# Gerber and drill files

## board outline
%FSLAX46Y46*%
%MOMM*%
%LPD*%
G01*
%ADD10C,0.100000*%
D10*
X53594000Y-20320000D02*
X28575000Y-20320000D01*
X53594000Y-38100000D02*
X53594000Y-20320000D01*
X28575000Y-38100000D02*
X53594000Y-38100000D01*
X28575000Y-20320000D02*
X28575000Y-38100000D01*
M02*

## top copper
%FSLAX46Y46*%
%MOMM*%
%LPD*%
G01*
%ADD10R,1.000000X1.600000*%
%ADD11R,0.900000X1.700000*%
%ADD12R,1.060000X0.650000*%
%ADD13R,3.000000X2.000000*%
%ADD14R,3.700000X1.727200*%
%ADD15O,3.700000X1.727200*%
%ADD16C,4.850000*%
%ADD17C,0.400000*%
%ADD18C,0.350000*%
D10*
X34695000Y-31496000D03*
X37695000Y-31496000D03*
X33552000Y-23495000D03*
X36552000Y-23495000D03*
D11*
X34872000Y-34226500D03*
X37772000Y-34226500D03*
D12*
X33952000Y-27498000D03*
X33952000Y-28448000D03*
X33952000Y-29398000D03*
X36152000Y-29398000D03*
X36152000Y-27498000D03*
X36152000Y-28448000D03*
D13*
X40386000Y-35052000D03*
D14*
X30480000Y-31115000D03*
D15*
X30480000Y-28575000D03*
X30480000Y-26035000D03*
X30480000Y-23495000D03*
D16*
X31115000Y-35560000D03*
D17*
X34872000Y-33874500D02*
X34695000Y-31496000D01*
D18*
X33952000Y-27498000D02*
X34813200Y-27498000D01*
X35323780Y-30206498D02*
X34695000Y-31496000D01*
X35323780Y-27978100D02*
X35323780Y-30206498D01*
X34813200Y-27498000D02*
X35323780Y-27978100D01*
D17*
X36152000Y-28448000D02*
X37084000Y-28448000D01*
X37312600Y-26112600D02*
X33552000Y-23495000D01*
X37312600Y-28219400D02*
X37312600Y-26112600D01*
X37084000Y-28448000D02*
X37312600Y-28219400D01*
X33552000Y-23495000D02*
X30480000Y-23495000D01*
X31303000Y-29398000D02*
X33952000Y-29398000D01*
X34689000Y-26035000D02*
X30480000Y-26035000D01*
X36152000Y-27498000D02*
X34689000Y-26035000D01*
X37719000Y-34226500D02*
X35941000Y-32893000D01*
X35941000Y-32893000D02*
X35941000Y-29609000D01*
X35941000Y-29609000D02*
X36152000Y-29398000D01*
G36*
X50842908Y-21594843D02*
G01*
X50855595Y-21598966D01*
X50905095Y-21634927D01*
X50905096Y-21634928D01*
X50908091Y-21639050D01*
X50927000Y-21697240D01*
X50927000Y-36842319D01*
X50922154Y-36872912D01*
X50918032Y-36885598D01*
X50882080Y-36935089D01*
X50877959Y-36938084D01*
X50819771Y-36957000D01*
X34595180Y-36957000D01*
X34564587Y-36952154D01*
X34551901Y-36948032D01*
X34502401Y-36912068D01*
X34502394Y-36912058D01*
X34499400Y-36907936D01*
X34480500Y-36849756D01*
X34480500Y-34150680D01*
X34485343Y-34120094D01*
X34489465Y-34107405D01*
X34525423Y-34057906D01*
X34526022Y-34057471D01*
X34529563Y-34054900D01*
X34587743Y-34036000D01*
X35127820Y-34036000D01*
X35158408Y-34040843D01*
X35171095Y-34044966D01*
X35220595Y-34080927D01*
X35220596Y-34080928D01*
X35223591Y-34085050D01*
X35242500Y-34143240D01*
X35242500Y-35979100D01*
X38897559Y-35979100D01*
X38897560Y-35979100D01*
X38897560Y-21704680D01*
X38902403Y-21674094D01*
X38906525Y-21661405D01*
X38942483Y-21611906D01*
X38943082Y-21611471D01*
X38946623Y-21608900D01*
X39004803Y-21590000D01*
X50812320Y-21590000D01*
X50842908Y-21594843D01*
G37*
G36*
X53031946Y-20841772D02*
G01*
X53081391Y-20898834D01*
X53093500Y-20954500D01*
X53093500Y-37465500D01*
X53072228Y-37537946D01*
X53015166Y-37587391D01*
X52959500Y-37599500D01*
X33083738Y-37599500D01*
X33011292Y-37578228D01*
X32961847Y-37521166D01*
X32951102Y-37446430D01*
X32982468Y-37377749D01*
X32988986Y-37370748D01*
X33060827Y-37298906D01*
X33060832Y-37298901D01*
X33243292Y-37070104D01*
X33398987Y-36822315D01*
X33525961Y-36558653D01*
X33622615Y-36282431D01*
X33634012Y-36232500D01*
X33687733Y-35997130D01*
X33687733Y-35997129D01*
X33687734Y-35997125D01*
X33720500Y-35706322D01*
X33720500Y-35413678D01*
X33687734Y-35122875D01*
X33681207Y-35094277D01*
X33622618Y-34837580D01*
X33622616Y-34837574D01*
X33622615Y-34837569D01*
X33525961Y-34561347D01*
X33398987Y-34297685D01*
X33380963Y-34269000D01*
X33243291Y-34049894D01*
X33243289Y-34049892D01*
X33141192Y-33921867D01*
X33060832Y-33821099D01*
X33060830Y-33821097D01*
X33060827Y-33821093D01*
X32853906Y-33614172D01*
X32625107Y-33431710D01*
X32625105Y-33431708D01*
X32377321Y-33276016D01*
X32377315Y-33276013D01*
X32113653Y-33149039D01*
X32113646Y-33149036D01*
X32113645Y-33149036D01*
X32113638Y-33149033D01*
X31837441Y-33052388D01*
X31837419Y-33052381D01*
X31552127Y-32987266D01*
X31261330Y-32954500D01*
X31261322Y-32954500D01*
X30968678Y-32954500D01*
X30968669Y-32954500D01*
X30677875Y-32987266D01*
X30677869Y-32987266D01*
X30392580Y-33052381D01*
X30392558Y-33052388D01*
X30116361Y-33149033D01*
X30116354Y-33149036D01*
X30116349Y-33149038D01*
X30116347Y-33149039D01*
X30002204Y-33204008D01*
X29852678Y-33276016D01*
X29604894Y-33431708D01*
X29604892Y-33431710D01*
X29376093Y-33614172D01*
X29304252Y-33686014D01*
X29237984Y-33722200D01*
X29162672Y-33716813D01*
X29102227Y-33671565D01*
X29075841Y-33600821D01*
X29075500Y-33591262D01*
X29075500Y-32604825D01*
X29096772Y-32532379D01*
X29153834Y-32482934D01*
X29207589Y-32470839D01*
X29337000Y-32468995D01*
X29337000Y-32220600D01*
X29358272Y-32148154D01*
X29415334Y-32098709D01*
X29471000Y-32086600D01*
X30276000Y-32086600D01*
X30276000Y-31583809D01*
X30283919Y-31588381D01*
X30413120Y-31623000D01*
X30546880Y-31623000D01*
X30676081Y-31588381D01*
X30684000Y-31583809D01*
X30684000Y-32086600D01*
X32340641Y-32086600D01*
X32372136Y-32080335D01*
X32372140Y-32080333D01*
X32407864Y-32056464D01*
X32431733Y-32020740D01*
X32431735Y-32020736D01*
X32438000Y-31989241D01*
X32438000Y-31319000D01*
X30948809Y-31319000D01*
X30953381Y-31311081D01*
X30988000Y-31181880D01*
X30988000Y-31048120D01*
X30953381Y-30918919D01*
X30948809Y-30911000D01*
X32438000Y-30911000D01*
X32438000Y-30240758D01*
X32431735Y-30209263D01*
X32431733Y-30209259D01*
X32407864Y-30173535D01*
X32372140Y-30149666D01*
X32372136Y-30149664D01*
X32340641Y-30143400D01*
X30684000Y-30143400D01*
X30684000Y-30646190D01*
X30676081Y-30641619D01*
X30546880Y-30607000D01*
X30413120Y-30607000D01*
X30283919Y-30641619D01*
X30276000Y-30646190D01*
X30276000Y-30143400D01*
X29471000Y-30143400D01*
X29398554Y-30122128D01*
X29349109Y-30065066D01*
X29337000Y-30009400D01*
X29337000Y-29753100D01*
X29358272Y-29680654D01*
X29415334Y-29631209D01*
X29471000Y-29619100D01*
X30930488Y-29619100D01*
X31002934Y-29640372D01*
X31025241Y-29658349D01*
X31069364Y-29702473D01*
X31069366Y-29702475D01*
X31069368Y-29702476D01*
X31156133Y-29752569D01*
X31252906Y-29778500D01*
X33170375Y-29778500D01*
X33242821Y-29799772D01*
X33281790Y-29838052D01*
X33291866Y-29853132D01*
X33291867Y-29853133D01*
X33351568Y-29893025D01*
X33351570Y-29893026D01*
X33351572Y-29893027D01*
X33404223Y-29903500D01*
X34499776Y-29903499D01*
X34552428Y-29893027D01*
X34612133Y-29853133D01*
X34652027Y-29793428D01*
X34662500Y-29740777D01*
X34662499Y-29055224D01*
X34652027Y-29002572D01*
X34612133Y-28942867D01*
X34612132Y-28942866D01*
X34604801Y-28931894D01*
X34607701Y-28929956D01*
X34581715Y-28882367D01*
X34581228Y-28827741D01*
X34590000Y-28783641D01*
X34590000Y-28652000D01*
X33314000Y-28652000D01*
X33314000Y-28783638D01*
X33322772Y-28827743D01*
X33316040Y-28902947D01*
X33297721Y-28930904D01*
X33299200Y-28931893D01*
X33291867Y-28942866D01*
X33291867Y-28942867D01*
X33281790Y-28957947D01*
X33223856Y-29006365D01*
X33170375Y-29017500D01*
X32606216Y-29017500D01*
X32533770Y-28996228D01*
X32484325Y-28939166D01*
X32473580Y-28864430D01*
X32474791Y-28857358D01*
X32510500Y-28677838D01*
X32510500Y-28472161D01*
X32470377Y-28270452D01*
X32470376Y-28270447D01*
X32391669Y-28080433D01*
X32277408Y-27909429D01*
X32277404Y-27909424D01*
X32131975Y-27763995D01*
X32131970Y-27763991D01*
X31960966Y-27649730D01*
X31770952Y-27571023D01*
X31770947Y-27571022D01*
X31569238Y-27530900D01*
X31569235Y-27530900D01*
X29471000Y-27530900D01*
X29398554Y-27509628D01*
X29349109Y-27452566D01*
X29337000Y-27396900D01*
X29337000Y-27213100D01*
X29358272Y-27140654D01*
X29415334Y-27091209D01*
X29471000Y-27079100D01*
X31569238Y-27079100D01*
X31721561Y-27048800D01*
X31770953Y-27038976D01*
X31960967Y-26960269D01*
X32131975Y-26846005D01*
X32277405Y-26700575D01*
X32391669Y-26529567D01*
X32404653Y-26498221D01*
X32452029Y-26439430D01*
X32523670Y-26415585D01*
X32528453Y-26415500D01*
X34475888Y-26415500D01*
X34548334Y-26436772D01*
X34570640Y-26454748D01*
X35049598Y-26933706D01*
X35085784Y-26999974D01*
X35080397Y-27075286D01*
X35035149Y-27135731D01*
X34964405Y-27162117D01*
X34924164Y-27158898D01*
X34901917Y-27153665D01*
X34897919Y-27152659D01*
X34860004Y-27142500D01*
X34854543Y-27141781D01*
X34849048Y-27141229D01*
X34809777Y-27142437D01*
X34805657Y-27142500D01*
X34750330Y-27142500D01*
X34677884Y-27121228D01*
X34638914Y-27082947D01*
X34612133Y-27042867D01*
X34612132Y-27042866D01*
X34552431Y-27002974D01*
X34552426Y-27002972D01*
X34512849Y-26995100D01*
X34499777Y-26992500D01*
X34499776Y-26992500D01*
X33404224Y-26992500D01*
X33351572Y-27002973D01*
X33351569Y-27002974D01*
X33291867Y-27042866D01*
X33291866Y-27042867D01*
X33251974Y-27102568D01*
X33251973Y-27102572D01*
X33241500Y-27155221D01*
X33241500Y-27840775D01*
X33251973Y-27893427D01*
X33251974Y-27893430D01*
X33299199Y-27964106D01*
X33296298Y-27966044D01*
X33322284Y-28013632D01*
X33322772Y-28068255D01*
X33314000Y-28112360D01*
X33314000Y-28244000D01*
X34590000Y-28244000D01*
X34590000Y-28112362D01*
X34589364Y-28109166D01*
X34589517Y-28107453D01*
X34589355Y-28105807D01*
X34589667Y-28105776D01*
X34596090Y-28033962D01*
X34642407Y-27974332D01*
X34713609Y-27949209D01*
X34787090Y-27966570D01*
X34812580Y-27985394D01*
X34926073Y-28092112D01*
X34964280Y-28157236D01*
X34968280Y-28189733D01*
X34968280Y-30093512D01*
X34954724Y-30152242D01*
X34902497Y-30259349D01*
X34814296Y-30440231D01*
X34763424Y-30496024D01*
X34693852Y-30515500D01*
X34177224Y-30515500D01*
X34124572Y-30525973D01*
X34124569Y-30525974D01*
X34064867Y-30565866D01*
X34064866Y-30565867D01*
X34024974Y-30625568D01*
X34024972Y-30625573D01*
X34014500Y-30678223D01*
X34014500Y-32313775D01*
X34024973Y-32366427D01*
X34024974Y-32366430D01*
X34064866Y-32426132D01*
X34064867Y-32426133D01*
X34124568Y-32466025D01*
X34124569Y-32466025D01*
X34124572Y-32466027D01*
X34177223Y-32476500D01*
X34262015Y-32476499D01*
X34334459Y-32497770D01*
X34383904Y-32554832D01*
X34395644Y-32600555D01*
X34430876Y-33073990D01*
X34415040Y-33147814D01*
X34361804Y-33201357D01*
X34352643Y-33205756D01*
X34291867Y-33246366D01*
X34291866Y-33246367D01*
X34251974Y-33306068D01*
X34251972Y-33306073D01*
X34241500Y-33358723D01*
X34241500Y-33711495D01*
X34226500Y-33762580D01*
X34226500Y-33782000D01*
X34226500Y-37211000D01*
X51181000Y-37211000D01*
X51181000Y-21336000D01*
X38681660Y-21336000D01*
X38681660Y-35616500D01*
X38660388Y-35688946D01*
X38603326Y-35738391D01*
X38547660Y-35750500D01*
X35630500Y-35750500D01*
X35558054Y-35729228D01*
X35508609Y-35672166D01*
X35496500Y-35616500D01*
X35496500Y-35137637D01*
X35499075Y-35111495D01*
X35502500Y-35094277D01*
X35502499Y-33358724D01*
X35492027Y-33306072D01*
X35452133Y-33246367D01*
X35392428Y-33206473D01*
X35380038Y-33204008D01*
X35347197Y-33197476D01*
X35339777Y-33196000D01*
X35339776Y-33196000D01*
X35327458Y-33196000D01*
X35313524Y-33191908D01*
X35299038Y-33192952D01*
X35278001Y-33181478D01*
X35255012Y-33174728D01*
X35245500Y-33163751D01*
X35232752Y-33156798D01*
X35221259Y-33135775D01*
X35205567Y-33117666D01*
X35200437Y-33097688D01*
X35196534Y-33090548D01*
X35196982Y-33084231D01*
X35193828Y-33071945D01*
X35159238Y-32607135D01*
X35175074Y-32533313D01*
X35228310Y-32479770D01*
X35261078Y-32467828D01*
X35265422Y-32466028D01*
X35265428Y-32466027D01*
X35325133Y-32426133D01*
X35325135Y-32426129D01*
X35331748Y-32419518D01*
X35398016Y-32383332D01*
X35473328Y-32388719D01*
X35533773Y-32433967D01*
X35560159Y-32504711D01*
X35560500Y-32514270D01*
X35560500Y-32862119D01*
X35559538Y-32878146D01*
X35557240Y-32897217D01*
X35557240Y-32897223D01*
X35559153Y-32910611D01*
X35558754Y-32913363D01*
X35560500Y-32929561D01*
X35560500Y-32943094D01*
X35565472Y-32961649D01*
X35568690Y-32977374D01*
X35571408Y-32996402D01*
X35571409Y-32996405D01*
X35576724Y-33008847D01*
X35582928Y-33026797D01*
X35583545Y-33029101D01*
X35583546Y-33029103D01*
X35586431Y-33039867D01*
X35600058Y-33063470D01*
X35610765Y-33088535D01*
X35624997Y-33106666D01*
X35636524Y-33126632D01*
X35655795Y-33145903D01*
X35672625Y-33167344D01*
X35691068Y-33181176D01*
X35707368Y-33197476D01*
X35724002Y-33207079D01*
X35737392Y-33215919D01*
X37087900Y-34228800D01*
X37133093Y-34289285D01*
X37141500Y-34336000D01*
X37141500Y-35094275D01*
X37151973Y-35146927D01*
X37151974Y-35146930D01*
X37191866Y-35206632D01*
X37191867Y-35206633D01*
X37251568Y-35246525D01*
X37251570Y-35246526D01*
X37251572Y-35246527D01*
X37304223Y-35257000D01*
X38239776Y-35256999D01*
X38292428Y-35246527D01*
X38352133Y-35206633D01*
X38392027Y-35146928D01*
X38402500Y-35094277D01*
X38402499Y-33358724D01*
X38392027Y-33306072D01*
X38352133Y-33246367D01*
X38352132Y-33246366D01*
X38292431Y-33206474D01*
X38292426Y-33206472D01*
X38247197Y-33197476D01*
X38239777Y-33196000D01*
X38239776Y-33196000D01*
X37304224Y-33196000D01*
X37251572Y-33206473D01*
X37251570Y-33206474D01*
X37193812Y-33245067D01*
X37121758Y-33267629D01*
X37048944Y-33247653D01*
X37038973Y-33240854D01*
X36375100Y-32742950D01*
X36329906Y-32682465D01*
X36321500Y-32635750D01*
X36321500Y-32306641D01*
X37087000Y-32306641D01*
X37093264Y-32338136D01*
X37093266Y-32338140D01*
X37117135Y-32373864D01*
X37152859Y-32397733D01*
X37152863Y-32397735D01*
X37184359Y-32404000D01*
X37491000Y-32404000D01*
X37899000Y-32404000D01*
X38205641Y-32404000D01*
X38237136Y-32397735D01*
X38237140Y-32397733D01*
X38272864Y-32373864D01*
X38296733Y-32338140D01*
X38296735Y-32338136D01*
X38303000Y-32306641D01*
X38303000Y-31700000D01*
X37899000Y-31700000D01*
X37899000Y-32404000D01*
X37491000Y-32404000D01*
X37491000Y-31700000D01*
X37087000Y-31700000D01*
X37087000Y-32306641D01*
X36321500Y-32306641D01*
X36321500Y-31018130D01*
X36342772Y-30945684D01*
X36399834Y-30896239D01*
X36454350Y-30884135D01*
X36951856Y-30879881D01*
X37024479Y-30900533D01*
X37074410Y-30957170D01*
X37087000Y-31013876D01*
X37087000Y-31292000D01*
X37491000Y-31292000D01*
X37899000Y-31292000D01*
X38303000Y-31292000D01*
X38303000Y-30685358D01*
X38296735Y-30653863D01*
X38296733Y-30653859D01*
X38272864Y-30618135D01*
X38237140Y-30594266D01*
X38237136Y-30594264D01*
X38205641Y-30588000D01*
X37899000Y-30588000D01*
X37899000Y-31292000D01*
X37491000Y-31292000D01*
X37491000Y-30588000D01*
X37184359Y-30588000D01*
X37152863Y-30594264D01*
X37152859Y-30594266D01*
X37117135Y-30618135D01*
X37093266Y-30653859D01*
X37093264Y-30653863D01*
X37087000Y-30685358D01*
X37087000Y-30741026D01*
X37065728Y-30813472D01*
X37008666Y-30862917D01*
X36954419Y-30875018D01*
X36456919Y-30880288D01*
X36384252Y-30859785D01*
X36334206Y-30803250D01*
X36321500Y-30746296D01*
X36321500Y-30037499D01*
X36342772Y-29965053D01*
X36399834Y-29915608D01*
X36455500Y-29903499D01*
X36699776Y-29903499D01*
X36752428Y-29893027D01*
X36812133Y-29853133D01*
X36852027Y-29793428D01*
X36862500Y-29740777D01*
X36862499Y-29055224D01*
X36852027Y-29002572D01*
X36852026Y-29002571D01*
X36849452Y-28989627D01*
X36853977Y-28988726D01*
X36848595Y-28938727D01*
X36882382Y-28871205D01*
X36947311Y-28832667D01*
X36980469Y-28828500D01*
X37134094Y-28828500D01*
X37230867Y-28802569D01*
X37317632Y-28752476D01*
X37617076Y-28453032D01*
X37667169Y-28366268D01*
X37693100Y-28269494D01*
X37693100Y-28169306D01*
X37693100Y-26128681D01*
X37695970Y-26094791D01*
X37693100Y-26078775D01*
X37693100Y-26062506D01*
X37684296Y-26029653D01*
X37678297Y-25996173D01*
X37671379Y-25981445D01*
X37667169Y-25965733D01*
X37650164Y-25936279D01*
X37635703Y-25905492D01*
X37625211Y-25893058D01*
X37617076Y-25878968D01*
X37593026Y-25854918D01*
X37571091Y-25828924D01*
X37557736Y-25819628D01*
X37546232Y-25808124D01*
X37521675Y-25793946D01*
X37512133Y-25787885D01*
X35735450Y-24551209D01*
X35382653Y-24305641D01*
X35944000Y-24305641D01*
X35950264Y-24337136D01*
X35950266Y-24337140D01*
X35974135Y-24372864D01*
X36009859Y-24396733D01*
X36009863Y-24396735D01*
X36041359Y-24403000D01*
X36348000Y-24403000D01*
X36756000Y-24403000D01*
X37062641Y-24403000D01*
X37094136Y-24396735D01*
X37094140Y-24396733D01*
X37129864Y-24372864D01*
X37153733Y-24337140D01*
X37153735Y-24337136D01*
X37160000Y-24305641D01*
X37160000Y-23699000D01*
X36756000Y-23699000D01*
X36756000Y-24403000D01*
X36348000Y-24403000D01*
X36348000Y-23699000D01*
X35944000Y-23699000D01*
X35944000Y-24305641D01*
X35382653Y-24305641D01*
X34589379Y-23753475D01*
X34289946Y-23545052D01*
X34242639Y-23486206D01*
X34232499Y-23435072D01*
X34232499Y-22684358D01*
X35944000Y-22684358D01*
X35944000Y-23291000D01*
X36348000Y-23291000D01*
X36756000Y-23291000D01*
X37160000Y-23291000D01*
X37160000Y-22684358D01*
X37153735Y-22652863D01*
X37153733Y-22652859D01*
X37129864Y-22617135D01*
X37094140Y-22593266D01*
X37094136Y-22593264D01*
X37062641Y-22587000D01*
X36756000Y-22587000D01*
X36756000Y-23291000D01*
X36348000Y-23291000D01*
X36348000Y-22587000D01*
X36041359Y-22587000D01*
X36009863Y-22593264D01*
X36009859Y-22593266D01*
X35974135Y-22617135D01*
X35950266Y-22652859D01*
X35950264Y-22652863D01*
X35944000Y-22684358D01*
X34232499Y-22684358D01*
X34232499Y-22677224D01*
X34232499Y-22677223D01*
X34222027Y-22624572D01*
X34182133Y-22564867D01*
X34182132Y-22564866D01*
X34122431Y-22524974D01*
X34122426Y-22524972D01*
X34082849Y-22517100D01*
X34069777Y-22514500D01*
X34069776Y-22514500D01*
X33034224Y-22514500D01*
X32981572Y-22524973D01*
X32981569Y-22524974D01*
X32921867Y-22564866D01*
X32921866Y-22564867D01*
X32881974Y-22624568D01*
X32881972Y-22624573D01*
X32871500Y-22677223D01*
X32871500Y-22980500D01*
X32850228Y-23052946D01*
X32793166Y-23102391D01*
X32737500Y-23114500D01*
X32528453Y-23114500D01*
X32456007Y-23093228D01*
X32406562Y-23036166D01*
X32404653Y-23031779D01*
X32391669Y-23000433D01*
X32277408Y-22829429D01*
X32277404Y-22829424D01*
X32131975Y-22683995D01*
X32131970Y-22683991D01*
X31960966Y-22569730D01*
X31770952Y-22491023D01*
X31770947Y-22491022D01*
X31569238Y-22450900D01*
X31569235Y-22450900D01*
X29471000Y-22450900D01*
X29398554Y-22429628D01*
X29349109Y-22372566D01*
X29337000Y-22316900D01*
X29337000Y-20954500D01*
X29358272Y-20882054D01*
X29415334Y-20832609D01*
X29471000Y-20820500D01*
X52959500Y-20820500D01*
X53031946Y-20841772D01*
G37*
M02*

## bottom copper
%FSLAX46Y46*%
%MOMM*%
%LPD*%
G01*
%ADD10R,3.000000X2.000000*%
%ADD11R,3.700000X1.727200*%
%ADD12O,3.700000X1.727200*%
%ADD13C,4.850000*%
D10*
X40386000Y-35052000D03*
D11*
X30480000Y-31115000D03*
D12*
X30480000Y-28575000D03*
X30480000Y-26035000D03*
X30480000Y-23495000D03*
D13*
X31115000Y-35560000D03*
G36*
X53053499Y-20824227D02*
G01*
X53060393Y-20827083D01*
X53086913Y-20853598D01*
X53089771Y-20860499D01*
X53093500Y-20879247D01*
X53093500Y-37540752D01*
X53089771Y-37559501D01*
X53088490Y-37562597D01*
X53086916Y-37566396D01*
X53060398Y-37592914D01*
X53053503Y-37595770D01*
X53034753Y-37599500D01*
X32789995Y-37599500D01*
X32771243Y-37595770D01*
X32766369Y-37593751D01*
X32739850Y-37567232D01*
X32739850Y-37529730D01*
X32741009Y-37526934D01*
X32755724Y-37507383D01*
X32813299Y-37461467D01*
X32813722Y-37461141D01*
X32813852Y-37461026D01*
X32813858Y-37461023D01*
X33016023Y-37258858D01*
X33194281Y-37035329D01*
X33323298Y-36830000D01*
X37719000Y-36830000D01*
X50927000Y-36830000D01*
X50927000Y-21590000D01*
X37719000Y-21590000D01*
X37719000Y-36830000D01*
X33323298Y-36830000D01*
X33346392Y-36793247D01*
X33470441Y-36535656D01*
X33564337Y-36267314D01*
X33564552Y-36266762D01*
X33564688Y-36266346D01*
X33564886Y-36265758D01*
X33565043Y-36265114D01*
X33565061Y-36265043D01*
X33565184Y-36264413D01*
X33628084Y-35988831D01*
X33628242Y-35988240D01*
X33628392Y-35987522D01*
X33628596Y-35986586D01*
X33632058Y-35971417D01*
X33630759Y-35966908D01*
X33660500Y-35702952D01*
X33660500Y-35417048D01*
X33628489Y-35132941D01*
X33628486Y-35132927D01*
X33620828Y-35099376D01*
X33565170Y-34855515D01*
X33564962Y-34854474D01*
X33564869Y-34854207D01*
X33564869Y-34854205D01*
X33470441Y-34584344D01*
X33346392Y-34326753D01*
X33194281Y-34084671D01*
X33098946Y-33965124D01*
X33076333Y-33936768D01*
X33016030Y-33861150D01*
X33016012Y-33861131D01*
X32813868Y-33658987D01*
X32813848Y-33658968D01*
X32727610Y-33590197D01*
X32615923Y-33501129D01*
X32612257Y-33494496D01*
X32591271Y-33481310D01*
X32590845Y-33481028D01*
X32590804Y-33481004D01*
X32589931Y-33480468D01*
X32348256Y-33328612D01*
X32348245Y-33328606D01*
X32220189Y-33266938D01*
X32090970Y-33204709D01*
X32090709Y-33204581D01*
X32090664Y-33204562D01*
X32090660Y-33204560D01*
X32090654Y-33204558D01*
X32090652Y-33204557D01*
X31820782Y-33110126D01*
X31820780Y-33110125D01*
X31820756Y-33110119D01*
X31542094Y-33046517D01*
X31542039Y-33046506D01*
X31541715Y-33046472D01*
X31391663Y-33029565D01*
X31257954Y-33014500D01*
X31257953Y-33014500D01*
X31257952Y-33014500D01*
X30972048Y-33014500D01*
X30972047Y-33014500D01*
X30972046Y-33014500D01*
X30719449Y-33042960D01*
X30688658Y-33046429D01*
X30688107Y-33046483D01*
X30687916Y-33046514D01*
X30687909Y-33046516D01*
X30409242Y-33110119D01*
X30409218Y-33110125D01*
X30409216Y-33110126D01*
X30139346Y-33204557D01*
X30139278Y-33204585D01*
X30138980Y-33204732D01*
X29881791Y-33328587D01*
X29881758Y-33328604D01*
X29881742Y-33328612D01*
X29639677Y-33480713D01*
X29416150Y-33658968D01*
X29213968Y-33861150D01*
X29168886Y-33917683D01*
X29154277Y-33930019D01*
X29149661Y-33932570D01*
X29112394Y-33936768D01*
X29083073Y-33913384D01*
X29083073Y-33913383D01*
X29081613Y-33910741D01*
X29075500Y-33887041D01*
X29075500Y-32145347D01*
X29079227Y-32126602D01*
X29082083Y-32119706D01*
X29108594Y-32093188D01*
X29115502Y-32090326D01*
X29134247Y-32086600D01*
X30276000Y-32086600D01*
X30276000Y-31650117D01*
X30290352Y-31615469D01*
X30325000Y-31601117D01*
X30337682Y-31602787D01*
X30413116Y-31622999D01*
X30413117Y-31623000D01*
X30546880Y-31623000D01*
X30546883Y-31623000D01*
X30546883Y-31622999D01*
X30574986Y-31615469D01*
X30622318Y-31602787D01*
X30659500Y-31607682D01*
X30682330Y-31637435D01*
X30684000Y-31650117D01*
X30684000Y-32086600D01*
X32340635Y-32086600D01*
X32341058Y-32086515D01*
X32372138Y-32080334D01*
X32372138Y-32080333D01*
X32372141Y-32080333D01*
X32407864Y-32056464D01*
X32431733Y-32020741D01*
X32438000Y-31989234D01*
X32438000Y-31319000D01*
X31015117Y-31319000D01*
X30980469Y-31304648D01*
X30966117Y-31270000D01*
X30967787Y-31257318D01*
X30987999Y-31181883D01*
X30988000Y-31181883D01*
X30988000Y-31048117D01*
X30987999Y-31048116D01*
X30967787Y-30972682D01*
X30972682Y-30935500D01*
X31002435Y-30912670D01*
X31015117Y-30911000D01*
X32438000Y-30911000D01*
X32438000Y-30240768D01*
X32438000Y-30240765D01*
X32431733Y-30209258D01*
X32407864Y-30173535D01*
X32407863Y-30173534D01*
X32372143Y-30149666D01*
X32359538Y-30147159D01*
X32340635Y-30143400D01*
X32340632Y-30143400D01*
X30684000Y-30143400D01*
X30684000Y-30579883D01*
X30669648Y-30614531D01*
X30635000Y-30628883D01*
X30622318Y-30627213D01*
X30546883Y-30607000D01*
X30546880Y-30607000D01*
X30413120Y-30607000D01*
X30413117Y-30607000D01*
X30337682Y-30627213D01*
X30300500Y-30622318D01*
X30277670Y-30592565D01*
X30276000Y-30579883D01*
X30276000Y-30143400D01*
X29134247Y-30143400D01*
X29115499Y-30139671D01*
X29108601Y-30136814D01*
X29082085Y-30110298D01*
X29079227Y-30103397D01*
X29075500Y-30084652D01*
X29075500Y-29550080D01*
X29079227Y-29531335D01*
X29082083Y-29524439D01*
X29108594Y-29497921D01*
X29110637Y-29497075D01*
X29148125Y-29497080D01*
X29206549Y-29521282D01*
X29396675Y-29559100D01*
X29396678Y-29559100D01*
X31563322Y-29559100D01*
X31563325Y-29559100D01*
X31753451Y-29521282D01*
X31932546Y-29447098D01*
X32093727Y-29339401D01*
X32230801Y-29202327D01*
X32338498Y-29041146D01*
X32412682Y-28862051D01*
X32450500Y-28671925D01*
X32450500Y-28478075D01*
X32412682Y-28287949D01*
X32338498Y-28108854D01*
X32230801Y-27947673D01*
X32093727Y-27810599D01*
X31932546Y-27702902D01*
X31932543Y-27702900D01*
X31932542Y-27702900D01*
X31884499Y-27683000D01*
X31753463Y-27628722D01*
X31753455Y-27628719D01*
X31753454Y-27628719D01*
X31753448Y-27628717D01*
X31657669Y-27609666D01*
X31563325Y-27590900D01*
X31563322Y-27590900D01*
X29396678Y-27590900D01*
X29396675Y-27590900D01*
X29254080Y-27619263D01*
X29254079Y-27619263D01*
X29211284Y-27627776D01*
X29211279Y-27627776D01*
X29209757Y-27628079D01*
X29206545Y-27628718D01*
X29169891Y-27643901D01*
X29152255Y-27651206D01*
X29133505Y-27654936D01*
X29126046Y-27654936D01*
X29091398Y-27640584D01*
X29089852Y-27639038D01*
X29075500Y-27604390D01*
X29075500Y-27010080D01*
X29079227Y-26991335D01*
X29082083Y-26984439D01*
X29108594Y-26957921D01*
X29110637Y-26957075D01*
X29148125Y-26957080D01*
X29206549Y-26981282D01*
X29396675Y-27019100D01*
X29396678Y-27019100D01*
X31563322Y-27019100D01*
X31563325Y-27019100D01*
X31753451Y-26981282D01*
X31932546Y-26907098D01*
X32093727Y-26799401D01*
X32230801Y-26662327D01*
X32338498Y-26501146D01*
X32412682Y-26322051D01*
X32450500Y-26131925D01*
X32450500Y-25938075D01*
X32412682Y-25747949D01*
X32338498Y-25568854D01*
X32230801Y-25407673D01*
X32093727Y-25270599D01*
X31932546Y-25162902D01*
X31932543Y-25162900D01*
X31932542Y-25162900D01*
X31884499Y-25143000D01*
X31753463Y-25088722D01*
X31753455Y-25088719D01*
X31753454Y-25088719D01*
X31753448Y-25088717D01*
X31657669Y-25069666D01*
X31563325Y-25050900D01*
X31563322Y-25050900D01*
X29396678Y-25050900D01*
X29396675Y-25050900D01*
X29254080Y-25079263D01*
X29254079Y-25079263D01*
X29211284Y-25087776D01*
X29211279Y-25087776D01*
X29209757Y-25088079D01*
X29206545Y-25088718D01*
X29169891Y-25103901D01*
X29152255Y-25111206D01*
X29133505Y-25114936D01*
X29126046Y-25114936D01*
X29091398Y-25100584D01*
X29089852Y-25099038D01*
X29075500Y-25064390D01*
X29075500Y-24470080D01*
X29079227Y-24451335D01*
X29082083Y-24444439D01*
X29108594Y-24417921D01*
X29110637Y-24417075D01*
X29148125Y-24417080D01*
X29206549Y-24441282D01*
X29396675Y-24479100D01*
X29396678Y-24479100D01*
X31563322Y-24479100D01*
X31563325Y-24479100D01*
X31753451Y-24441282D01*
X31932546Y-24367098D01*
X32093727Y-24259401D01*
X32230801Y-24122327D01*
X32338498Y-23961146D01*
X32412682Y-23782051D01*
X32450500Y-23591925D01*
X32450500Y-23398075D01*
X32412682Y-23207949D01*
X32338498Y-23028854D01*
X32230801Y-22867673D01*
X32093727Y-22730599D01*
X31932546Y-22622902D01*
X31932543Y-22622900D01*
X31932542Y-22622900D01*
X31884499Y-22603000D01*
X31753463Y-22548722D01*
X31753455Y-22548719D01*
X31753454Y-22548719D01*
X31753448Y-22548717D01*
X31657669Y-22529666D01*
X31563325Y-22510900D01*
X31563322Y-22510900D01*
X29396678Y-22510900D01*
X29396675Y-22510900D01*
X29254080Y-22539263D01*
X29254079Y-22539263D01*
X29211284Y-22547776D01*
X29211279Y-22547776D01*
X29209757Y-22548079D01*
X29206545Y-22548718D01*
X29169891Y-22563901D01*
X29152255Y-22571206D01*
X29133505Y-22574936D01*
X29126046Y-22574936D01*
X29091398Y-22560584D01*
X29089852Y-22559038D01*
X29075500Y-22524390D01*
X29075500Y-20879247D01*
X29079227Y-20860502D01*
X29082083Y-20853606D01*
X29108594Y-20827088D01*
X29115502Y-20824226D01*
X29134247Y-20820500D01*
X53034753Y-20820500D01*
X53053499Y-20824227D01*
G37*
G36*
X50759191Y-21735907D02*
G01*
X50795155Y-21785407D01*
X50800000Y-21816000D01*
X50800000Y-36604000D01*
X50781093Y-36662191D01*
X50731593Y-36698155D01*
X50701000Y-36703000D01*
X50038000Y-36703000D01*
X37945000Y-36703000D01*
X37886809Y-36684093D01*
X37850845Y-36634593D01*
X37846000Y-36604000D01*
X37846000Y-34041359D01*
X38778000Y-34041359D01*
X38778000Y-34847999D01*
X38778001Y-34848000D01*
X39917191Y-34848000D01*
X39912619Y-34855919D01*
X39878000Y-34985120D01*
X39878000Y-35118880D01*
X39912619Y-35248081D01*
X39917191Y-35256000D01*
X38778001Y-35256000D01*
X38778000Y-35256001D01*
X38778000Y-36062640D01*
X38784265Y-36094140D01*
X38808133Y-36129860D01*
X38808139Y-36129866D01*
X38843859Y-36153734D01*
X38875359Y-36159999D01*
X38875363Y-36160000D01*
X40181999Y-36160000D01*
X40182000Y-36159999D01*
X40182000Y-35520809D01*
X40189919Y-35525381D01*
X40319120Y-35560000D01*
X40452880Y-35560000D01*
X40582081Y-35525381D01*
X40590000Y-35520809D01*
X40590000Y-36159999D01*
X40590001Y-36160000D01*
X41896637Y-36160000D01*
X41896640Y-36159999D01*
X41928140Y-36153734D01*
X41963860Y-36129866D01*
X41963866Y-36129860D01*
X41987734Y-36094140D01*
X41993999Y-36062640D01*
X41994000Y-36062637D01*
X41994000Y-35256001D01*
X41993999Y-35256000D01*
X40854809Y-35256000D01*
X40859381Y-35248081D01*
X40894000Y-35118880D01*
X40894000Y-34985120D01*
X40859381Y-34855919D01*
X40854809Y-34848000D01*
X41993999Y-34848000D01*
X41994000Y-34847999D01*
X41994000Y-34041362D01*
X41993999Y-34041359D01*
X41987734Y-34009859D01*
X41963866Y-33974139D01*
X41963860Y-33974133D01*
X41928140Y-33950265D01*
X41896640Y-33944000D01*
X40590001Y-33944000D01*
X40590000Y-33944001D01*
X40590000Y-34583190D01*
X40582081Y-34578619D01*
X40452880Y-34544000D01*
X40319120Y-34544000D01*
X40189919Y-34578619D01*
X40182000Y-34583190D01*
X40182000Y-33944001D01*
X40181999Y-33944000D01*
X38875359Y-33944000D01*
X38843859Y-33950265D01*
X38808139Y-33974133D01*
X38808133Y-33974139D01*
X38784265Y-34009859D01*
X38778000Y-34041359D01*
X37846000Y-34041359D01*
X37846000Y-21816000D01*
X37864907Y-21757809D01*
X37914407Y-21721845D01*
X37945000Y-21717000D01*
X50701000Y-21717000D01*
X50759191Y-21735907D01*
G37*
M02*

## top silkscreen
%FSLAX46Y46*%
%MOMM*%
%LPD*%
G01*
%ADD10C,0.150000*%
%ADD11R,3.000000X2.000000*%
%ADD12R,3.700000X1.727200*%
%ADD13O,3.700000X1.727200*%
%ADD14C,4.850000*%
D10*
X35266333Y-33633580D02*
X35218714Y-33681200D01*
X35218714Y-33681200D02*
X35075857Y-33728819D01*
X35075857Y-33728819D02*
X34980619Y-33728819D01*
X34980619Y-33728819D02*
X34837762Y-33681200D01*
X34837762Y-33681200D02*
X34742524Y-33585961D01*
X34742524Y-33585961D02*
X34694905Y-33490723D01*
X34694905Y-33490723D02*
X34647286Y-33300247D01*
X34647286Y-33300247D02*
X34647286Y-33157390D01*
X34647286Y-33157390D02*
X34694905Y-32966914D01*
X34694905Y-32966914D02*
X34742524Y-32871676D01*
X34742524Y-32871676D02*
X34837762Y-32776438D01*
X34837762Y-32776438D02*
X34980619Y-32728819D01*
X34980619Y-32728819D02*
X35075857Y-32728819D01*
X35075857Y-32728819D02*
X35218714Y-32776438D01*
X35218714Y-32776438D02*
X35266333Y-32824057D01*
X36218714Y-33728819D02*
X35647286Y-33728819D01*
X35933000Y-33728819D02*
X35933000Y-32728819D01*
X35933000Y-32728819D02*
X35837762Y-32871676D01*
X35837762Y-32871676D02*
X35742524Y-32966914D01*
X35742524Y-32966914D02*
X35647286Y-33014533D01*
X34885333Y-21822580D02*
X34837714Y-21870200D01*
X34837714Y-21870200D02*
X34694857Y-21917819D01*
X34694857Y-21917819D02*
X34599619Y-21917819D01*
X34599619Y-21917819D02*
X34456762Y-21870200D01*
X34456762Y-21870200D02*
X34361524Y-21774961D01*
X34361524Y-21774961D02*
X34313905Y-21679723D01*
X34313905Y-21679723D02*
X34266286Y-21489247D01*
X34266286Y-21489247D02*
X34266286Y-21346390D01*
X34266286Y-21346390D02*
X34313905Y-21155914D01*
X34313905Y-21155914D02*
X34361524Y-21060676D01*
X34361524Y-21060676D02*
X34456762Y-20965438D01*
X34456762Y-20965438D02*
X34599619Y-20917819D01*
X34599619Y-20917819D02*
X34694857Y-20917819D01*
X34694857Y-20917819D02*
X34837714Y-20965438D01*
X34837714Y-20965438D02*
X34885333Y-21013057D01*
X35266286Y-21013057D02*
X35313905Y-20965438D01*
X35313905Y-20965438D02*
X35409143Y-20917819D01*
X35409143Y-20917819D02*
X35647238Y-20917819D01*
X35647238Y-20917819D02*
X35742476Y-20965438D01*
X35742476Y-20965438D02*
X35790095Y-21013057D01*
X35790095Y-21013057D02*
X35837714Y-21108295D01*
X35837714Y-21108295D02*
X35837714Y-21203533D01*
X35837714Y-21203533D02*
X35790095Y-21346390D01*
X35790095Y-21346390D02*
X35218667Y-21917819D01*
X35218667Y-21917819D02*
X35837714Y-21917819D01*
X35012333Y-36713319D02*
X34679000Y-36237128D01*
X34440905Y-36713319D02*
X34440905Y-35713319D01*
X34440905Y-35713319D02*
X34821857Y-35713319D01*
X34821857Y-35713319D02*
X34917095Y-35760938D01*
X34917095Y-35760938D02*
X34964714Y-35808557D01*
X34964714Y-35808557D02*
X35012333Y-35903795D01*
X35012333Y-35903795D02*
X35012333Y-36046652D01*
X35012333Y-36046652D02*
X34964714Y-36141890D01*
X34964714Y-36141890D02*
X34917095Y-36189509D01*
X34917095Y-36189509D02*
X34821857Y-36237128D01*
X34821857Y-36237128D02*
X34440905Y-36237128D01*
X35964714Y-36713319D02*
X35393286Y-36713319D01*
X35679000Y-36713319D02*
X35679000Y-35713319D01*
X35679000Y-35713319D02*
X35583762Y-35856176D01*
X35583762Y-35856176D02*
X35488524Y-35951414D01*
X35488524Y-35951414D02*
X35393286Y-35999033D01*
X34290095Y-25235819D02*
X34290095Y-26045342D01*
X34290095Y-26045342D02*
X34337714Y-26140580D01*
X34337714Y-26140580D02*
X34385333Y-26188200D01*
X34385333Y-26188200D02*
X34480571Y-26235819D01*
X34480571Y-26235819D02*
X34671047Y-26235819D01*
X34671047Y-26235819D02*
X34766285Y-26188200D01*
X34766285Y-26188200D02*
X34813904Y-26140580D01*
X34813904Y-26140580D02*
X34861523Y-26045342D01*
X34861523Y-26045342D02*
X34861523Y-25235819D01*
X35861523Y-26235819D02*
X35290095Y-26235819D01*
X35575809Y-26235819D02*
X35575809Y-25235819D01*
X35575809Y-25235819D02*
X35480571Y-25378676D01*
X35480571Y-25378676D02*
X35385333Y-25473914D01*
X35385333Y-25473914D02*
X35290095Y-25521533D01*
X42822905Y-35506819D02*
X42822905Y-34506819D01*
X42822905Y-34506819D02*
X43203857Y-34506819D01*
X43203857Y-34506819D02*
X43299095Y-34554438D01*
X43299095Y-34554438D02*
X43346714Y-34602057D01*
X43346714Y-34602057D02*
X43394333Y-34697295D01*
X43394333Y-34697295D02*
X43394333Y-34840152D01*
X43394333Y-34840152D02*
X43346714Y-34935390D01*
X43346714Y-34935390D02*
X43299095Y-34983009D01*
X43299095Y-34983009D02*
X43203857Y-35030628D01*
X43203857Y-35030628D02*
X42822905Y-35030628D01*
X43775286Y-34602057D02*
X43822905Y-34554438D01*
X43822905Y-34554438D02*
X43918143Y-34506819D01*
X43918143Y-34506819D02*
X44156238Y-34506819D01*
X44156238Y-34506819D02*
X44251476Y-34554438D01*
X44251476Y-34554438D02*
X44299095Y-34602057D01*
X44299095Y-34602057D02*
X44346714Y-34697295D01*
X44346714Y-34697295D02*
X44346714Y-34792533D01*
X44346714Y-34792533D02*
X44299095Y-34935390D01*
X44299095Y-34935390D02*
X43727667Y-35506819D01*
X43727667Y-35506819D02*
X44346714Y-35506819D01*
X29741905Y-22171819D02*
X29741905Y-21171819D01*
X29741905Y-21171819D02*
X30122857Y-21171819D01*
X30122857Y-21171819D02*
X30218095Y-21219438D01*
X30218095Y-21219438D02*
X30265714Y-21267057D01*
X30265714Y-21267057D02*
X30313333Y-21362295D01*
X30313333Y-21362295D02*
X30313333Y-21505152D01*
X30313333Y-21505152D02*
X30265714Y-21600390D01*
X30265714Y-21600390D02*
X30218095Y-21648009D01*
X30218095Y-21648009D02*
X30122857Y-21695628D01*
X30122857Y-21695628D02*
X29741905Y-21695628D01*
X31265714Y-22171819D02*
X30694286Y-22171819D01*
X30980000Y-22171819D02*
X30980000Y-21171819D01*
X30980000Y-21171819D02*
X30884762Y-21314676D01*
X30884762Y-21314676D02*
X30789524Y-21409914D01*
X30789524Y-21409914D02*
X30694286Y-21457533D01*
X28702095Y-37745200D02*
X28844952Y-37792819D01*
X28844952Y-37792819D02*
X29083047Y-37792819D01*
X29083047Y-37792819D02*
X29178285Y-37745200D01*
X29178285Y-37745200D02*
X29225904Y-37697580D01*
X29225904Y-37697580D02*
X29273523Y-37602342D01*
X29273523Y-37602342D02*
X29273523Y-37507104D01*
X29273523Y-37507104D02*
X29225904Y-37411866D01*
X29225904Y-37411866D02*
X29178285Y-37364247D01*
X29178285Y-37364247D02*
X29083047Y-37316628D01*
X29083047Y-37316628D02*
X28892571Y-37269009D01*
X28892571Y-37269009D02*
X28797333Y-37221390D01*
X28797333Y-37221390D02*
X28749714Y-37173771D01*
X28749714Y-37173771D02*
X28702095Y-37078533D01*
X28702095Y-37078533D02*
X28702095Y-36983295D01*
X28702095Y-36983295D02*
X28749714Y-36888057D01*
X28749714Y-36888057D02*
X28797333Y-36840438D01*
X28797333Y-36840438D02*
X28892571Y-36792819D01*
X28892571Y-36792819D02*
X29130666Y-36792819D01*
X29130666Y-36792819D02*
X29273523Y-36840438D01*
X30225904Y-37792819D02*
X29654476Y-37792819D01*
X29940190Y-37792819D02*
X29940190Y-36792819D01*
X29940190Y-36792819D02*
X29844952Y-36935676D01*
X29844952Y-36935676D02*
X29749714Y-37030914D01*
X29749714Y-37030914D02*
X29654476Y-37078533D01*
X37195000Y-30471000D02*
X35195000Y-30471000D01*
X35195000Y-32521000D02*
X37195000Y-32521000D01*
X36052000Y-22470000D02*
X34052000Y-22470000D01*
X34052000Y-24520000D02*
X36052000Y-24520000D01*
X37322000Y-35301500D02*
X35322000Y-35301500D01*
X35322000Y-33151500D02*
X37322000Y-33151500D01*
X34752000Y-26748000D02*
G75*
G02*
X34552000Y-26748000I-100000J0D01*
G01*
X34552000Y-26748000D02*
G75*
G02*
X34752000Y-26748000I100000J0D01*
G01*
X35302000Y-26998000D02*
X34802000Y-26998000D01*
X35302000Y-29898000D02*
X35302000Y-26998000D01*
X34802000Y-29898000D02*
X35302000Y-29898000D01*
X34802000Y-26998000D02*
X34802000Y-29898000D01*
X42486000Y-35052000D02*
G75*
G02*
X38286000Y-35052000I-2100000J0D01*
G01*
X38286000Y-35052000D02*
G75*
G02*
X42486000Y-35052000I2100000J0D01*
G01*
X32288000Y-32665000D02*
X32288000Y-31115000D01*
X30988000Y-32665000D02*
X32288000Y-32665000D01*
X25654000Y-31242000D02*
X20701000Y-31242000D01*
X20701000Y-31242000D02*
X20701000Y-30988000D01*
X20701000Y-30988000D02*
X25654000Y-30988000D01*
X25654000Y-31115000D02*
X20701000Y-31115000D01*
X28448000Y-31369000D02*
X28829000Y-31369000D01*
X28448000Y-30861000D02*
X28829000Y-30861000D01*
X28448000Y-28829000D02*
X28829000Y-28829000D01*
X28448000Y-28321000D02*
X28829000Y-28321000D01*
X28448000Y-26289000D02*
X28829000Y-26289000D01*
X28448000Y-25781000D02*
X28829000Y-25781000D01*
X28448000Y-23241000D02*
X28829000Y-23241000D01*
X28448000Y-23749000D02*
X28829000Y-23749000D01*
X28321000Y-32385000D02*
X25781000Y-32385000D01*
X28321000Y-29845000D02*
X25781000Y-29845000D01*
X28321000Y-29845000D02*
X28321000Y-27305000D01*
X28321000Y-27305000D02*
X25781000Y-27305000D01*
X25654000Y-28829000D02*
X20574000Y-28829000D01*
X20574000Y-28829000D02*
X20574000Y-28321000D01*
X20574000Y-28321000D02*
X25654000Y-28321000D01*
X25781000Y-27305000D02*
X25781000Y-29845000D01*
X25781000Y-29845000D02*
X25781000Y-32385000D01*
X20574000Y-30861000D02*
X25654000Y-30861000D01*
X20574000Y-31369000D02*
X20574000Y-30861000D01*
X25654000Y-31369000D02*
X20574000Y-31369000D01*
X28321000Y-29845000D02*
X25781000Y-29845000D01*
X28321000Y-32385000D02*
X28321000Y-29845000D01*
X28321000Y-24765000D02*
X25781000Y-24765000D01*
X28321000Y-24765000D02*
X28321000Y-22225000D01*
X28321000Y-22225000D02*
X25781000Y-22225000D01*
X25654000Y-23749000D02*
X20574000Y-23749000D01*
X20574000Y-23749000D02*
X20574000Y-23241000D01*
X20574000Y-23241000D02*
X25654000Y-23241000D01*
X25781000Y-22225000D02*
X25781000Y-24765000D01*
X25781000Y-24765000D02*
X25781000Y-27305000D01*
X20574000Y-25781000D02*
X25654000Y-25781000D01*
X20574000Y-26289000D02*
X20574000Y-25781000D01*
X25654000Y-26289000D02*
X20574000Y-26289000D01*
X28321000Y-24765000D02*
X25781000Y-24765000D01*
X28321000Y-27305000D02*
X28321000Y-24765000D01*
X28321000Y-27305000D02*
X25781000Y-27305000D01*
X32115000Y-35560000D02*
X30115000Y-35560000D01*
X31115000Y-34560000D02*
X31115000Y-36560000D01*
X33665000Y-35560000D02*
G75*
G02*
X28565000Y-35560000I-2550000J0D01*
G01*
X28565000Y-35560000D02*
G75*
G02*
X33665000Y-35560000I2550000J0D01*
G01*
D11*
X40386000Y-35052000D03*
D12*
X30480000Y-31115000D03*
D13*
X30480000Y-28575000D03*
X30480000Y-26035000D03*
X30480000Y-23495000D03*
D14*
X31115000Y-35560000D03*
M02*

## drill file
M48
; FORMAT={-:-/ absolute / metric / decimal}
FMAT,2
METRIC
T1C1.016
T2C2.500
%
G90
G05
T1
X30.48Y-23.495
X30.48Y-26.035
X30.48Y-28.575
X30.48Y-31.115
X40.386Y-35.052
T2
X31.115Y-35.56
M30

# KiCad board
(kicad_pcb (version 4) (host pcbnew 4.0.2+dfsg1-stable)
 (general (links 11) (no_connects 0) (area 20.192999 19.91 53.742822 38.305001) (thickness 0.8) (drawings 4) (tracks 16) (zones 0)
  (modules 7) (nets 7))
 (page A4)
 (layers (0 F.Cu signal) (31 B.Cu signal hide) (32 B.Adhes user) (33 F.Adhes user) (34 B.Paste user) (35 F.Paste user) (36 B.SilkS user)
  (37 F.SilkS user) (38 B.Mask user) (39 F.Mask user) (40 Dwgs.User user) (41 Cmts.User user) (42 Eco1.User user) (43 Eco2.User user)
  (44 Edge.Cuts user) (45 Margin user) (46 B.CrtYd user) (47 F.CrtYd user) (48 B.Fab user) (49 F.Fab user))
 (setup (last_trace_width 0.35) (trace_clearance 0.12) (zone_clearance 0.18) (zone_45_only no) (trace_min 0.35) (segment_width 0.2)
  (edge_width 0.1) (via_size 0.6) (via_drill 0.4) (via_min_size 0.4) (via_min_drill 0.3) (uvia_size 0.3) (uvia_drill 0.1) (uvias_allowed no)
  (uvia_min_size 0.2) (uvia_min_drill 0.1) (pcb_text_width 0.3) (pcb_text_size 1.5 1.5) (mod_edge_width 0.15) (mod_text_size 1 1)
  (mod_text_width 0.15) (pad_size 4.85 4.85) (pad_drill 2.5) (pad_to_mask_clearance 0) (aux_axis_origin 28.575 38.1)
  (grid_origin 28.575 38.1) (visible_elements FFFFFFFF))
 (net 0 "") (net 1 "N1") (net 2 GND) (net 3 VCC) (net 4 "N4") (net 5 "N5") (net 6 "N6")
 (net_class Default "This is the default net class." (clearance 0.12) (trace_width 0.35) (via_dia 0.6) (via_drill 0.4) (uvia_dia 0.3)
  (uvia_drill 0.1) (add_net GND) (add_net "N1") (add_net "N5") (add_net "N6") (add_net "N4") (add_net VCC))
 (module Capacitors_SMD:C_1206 (layer F.Cu) (at 36.195 31.496)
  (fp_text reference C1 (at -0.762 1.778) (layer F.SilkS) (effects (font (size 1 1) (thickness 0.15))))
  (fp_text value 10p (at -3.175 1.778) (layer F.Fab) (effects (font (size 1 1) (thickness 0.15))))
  (fp_line (start 1 -1.025) (end -1 -1.025) (layer F.SilkS) (width 0.15))
  (fp_line (start -1 1.025) (end 1 1.025) (layer F.SilkS) (width 0.15))
  (pad 1 smd rect (at -1.5 0) (size 1 1.6) (layers F.Cu F.Paste F.Mask) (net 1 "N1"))
  (pad 2 smd rect (at 1.5 0) (size 1 1.6) (layers F.Cu F.Paste F.Mask) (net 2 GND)))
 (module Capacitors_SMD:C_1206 (layer F.Cu) (at 35.052 23.495)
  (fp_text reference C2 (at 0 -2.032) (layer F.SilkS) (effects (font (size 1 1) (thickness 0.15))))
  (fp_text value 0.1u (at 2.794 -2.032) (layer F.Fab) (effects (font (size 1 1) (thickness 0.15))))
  (fp_line (start 1 -1.025) (end -1 -1.025) (layer F.SilkS) (width 0.15))
  (fp_line (start -1 1.025) (end 1 1.025) (layer F.SilkS) (width 0.15))
  (pad 1 smd rect (at -1.5 0) (size 1 1.6) (layers F.Cu F.Paste F.Mask) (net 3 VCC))
  (pad 2 smd rect (at 1.5 0) (size 1 1.6) (layers F.Cu F.Paste F.Mask) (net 2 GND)))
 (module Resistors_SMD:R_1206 (layer F.Cu) (at 36.322 34.2265)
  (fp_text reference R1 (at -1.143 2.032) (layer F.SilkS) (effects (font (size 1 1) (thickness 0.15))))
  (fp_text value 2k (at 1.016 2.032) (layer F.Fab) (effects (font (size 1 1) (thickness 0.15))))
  (fp_line (start 1 1.075) (end -1 1.075) (layer F.SilkS) (width 0.15))
  (fp_line (start -1 -1.075) (end 1 -1.075) (layer F.SilkS) (width 0.15))
  (pad 1 smd rect (at -1.45 0) (size 0.9 1.7) (layers F.Cu F.Paste F.Mask) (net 1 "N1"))
  (pad 2 smd rect (at 1.45 0) (size 0.9 1.7) (layers F.Cu F.Paste F.Mask) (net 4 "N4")))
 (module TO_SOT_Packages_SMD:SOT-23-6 (layer F.Cu) (at 35.052 28.448)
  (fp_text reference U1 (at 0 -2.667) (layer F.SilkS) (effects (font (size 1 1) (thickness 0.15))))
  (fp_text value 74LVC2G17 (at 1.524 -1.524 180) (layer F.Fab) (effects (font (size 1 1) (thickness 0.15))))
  (fp_circle (center -0.4 -1.7) (end -0.3 -1.7) (layer F.SilkS) (width 0.15))
  (fp_line (start 0.25 -1.45) (end -0.25 -1.45) (layer F.SilkS) (width 0.15))
  (fp_line (start 0.25 1.45) (end 0.25 -1.45) (layer F.SilkS) (width 0.15))
  (fp_line (start -0.25 1.45) (end 0.25 1.45) (layer F.SilkS) (width 0.15))
  (fp_line (start -0.25 -1.45) (end -0.25 1.45) (layer F.SilkS) (width 0.15))
  (pad 1 smd rect (at -1.1 -0.95) (size 1.06 0.65) (layers F.Cu F.Paste F.Mask) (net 1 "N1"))
  (pad 2 smd rect (at -1.1 0) (size 1.06 0.65) (layers F.Cu F.Paste F.Mask) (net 2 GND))
  (pad 3 smd rect (at -1.1 0.95) (size 1.06 0.65) (layers F.Cu F.Paste F.Mask) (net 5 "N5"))
  (pad 4 smd rect (at 1.1 0.95) (size 1.06 0.65) (layers F.Cu F.Paste F.Mask) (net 4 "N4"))
  (pad 6 smd rect (at 1.1 -0.95) (size 1.06 0.65) (layers F.Cu F.Paste F.Mask) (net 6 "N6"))
  (pad 5 smd rect (at 1.1 0) (size 1.06 0.65) (layers F.Cu F.Paste F.Mask) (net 3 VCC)))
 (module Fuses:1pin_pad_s (layer F.Cu) (at 40.386 35.052)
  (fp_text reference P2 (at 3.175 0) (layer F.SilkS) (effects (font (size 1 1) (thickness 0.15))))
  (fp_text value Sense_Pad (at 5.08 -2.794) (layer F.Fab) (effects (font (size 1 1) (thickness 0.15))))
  (fp_circle (center 0 0) (end 0 -2.1) (layer F.SilkS) (width 0.15))
  (pad 1 thru_hole rect (at 0 0) (size 3 2) (drill 1.016) (layers *.Cu *.Mask F.SilkS) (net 1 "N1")))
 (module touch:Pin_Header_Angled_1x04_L (layer F.Cu) (at 30.48 31.115 180)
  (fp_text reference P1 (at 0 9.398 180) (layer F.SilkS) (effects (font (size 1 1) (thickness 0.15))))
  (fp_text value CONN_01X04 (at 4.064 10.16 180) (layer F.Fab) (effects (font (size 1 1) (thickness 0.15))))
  (fp_line (start -1.808 -1.55) (end -1.808 0) (layer F.SilkS) (width 0.15))
  (fp_line (start -0.508 -1.55) (end -1.808 -1.55) (layer F.SilkS) (width 0.15))
  (fp_line (start 4.826 -0.127) (end 9.779 -0.127) (layer F.SilkS) (width 0.15))
  (fp_line (start 9.779 -0.127) (end 9.779 0.127) (layer F.SilkS) (width 0.15))
  (fp_line (start 9.779 0.127) (end 4.826 0.127) (layer F.SilkS) (width 0.15))
  (fp_line (start 4.826 0) (end 9.779 0) (layer F.SilkS) (width 0.15))
  (fp_line (start 2.032 -0.254) (end 1.651 -0.254) (layer F.SilkS) (width 0.15))
  (fp_line (start 2.032 0.254) (end 1.651 0.254) (layer F.SilkS) (width 0.15))
  (fp_line (start 2.032 2.286) (end 1.651 2.286) (layer F.SilkS) (width 0.15))
  (fp_line (start 2.032 2.794) (end 1.651 2.794) (layer F.SilkS) (width 0.15))
  (fp_line (start 2.032 4.826) (end 1.651 4.826) (layer F.SilkS) (width 0.15))
  (fp_line (start 2.032 5.334) (end 1.651 5.334) (layer F.SilkS) (width 0.15))
  (fp_line (start 2.032 7.874) (end 1.651 7.874) (layer F.SilkS) (width 0.15))
  (fp_line (start 2.032 7.366) (end 1.651 7.366) (layer F.SilkS) (width 0.15))
  (fp_line (start 2.159 -1.27) (end 4.699 -1.27) (layer F.SilkS) (width 0.15))
  (fp_line (start 2.159 1.27) (end 4.699 1.27) (layer F.SilkS) (width 0.15))
  (fp_line (start 2.159 1.27) (end 2.159 3.81) (layer F.SilkS) (width 0.15))
  (fp_line (start 2.159 3.81) (end 4.699 3.81) (layer F.SilkS) (width 0.15))
  (fp_line (start 4.826 2.286) (end 9.906 2.286) (layer F.SilkS) (width 0.15))
  (fp_line (start 9.906 2.286) (end 9.906 2.794) (layer F.SilkS) (width 0.15))
  (fp_line (start 9.906 2.794) (end 4.826 2.794) (layer F.SilkS) (width 0.15))
  (fp_line (start 4.699 3.81) (end 4.699 1.27) (layer F.SilkS) (width 0.15))
  (fp_line (start 4.699 1.27) (end 4.699 -1.27) (layer F.SilkS) (width 0.15))
  (fp_line (start 9.906 0.254) (end 4.826 0.254) (layer F.SilkS) (width 0.15))
  (fp_line (start 9.906 -0.254) (end 9.906 0.254) (layer F.SilkS) (width 0.15))
  (fp_line (start 4.826 -0.254) (end 9.906 -0.254) (layer F.SilkS) (width 0.15))
  (fp_line (start 2.159 1.27) (end 4.699 1.27) (layer F.SilkS) (width 0.15))
  (fp_line (start 2.159 -1.27) (end 2.159 1.27) (layer F.SilkS) (width 0.15))
  (fp_line (start 2.159 6.35) (end 4.699 6.35) (layer F.SilkS) (width 0.15))
  (fp_line (start 2.159 6.35) (end 2.159 8.89) (layer F.SilkS) (width 0.15))
  (fp_line (start 2.159 8.89) (end 4.699 8.89) (layer F.SilkS) (width 0.15))
  (fp_line (start 4.826 7.366) (end 9.906 7.366) (layer F.SilkS) (width 0.15))
  (fp_line (start 9.906 7.366) (end 9.906 7.874) (layer F.SilkS) (width 0.15))
  (fp_line (start 9.906 7.874) (end 4.826 7.874) (layer F.SilkS) (width 0.15))
  (fp_line (start 4.699 8.89) (end 4.699 6.35) (layer F.SilkS) (width 0.15))
  (fp_line (start 4.699 6.35) (end 4.699 3.81) (layer F.SilkS) (width 0.15))
  (fp_line (start 9.906 5.334) (end 4.826 5.334) (layer F.SilkS) (width 0.15))
  (fp_line (start 9.906 4.826) (end 9.906 5.334) (layer F.SilkS) (width 0.15))
  (fp_line (start 4.826 4.826) (end 9.906 4.826) (layer F.SilkS) (width 0.15))
  (fp_line (start 2.159 6.35) (end 4.699 6.35) (layer F.SilkS) (width 0.15))
  (fp_line (start 2.159 3.81) (end 2.159 6.35) (layer F.SilkS) (width 0.15))
  (fp_line (start 2.159 3.81) (end 4.699 3.81) (layer F.SilkS) (width 0.15))
  (pad 1 thru_hole rect (at 0 0 180) (size 3.7 1.7272) (drill 1.016) (layers *.Cu *.Mask F.SilkS) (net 2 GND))
  (pad 2 thru_hole oval (at 0 2.54 180) (size 3.7 1.7272) (drill 1.016) (layers *.Cu *.Mask F.SilkS) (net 5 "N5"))
  (pad 3 thru_hole oval (at 0 5.08 180) (size 3.7 1.7272) (drill 1.016) (layers *.Cu *.Mask F.SilkS) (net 6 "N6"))
  (pad 4 thru_hole oval (at 0 7.62 180) (size 3.7 1.7272) (drill 1.016) (layers *.Cu *.Mask F.SilkS) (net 3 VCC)))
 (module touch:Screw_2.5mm (layer F.Cu) (at 31.115 35.56)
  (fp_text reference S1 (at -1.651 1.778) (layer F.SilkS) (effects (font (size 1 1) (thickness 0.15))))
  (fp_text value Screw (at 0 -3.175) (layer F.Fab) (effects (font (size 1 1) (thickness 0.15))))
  (fp_line (start 1 0) (end -1 0) (layer F.SilkS) (width 0.15))
  (fp_line (start 0 -1) (end 0 1) (layer F.SilkS) (width 0.15))
  (fp_circle (center 0 0) (end 0 -2.55) (layer F.SilkS) (width 0.15))
  (pad 1 thru_hole circle (at 0 0) (size 4.85 4.85) (drill 2.5) (layers *.Cu *.Mask F.SilkS)))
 (gr_line (start 53.594 20.32) (end 28.575 20.32) (angle 90) (layer Edge.Cuts) (width 0.1))
 (gr_line (start 53.594 38.1) (end 53.594 20.32) (angle 90) (layer Edge.Cuts) (width 0.1))
 (gr_line (start 28.575 38.1) (end 53.594 38.1) (angle 90) (layer Edge.Cuts) (width 0.1))
 (gr_line (start 28.575 20.32) (end 28.575 38.1) (angle 90) (layer Edge.Cuts) (width 0.1))
 (segment (start 34.872 33.8745) (end 34.695 31.496) (width 0.4) (layer F.Cu) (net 1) (status 10))
 (segment (start 33.952 27.498) (end 34.8132 27.498) (width 0.35) (layer F.Cu) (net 1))
 (segment (start 35.32378 30.206498) (end 34.695 31.496) (width 0.35) (layer F.Cu) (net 1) (status 20))
 (segment (start 35.32378 27.9781) (end 35.32378 30.206498) (width 0.35) (layer F.Cu) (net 1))
 (segment (start 34.8132 27.498) (end 35.32378 27.9781) (width 0.35) (layer F.Cu) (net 1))
 (segment (start 36.152 28.448) (end 37.084 28.448) (width 0.4) (layer F.Cu) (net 3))
 (segment (start 37.3126 26.1126) (end 33.552 23.495) (width 0.4) (layer F.Cu) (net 3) (status 20))
 (segment (start 37.3126 28.2194) (end 37.3126 26.1126) (width 0.4) (layer F.Cu) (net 3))
 (segment (start 37.084 28.448) (end 37.3126 28.2194) (width 0.4) (layer F.Cu) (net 3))
 (segment (start 33.552 23.495) (end 30.48 23.495) (width 0.4) (layer F.Cu) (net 3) (status 10))
 (segment (start 31.303 29.398) (end 33.952 29.398) (width 0.4) (layer F.Cu) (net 5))
 (segment (start 34.689 26.035) (end 30.48 26.035) (width 0.4) (layer F.Cu) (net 6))
 (segment (start 36.152 27.498) (end 34.689 26.035) (width 0.4) (layer F.Cu) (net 6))
 (segment (start 37.719 34.2265) (end 35.941 32.893) (width 0.4) (layer F.Cu) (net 4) (status 10))
 (segment (start 35.941 32.893) (end 35.941 29.609) (width 0.4) (layer F.Cu) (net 4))
 (segment (start 35.941 29.609) (end 36.152 29.398) (width 0.4) (layer F.Cu) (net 4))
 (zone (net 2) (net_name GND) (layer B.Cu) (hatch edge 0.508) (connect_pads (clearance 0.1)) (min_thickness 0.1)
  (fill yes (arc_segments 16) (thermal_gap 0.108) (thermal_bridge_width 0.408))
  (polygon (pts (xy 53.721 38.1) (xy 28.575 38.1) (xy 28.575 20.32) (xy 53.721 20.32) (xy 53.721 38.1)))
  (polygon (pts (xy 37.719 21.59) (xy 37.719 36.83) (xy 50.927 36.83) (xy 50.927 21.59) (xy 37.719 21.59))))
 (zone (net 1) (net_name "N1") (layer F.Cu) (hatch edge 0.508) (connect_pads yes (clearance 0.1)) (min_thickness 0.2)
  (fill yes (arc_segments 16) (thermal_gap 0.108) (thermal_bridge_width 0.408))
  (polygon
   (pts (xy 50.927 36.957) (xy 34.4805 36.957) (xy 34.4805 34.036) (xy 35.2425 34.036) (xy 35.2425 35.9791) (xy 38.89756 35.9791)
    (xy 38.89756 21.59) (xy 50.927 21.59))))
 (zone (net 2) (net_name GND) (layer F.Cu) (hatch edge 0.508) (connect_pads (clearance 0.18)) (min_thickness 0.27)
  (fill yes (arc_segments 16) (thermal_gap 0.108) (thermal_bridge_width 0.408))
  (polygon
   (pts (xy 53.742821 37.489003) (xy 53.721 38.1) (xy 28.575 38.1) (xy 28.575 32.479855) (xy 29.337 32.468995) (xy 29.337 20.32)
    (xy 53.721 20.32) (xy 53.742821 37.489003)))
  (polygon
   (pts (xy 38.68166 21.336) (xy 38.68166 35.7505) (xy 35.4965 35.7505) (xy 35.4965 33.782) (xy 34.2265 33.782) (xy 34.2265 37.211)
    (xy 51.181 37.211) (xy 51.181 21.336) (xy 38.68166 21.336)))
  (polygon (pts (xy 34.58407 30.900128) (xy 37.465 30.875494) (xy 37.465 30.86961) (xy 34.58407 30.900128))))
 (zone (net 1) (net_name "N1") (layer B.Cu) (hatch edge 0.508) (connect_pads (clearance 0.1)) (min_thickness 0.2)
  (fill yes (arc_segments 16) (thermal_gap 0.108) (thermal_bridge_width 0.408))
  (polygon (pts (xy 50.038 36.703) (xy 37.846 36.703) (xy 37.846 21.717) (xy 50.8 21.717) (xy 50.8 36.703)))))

